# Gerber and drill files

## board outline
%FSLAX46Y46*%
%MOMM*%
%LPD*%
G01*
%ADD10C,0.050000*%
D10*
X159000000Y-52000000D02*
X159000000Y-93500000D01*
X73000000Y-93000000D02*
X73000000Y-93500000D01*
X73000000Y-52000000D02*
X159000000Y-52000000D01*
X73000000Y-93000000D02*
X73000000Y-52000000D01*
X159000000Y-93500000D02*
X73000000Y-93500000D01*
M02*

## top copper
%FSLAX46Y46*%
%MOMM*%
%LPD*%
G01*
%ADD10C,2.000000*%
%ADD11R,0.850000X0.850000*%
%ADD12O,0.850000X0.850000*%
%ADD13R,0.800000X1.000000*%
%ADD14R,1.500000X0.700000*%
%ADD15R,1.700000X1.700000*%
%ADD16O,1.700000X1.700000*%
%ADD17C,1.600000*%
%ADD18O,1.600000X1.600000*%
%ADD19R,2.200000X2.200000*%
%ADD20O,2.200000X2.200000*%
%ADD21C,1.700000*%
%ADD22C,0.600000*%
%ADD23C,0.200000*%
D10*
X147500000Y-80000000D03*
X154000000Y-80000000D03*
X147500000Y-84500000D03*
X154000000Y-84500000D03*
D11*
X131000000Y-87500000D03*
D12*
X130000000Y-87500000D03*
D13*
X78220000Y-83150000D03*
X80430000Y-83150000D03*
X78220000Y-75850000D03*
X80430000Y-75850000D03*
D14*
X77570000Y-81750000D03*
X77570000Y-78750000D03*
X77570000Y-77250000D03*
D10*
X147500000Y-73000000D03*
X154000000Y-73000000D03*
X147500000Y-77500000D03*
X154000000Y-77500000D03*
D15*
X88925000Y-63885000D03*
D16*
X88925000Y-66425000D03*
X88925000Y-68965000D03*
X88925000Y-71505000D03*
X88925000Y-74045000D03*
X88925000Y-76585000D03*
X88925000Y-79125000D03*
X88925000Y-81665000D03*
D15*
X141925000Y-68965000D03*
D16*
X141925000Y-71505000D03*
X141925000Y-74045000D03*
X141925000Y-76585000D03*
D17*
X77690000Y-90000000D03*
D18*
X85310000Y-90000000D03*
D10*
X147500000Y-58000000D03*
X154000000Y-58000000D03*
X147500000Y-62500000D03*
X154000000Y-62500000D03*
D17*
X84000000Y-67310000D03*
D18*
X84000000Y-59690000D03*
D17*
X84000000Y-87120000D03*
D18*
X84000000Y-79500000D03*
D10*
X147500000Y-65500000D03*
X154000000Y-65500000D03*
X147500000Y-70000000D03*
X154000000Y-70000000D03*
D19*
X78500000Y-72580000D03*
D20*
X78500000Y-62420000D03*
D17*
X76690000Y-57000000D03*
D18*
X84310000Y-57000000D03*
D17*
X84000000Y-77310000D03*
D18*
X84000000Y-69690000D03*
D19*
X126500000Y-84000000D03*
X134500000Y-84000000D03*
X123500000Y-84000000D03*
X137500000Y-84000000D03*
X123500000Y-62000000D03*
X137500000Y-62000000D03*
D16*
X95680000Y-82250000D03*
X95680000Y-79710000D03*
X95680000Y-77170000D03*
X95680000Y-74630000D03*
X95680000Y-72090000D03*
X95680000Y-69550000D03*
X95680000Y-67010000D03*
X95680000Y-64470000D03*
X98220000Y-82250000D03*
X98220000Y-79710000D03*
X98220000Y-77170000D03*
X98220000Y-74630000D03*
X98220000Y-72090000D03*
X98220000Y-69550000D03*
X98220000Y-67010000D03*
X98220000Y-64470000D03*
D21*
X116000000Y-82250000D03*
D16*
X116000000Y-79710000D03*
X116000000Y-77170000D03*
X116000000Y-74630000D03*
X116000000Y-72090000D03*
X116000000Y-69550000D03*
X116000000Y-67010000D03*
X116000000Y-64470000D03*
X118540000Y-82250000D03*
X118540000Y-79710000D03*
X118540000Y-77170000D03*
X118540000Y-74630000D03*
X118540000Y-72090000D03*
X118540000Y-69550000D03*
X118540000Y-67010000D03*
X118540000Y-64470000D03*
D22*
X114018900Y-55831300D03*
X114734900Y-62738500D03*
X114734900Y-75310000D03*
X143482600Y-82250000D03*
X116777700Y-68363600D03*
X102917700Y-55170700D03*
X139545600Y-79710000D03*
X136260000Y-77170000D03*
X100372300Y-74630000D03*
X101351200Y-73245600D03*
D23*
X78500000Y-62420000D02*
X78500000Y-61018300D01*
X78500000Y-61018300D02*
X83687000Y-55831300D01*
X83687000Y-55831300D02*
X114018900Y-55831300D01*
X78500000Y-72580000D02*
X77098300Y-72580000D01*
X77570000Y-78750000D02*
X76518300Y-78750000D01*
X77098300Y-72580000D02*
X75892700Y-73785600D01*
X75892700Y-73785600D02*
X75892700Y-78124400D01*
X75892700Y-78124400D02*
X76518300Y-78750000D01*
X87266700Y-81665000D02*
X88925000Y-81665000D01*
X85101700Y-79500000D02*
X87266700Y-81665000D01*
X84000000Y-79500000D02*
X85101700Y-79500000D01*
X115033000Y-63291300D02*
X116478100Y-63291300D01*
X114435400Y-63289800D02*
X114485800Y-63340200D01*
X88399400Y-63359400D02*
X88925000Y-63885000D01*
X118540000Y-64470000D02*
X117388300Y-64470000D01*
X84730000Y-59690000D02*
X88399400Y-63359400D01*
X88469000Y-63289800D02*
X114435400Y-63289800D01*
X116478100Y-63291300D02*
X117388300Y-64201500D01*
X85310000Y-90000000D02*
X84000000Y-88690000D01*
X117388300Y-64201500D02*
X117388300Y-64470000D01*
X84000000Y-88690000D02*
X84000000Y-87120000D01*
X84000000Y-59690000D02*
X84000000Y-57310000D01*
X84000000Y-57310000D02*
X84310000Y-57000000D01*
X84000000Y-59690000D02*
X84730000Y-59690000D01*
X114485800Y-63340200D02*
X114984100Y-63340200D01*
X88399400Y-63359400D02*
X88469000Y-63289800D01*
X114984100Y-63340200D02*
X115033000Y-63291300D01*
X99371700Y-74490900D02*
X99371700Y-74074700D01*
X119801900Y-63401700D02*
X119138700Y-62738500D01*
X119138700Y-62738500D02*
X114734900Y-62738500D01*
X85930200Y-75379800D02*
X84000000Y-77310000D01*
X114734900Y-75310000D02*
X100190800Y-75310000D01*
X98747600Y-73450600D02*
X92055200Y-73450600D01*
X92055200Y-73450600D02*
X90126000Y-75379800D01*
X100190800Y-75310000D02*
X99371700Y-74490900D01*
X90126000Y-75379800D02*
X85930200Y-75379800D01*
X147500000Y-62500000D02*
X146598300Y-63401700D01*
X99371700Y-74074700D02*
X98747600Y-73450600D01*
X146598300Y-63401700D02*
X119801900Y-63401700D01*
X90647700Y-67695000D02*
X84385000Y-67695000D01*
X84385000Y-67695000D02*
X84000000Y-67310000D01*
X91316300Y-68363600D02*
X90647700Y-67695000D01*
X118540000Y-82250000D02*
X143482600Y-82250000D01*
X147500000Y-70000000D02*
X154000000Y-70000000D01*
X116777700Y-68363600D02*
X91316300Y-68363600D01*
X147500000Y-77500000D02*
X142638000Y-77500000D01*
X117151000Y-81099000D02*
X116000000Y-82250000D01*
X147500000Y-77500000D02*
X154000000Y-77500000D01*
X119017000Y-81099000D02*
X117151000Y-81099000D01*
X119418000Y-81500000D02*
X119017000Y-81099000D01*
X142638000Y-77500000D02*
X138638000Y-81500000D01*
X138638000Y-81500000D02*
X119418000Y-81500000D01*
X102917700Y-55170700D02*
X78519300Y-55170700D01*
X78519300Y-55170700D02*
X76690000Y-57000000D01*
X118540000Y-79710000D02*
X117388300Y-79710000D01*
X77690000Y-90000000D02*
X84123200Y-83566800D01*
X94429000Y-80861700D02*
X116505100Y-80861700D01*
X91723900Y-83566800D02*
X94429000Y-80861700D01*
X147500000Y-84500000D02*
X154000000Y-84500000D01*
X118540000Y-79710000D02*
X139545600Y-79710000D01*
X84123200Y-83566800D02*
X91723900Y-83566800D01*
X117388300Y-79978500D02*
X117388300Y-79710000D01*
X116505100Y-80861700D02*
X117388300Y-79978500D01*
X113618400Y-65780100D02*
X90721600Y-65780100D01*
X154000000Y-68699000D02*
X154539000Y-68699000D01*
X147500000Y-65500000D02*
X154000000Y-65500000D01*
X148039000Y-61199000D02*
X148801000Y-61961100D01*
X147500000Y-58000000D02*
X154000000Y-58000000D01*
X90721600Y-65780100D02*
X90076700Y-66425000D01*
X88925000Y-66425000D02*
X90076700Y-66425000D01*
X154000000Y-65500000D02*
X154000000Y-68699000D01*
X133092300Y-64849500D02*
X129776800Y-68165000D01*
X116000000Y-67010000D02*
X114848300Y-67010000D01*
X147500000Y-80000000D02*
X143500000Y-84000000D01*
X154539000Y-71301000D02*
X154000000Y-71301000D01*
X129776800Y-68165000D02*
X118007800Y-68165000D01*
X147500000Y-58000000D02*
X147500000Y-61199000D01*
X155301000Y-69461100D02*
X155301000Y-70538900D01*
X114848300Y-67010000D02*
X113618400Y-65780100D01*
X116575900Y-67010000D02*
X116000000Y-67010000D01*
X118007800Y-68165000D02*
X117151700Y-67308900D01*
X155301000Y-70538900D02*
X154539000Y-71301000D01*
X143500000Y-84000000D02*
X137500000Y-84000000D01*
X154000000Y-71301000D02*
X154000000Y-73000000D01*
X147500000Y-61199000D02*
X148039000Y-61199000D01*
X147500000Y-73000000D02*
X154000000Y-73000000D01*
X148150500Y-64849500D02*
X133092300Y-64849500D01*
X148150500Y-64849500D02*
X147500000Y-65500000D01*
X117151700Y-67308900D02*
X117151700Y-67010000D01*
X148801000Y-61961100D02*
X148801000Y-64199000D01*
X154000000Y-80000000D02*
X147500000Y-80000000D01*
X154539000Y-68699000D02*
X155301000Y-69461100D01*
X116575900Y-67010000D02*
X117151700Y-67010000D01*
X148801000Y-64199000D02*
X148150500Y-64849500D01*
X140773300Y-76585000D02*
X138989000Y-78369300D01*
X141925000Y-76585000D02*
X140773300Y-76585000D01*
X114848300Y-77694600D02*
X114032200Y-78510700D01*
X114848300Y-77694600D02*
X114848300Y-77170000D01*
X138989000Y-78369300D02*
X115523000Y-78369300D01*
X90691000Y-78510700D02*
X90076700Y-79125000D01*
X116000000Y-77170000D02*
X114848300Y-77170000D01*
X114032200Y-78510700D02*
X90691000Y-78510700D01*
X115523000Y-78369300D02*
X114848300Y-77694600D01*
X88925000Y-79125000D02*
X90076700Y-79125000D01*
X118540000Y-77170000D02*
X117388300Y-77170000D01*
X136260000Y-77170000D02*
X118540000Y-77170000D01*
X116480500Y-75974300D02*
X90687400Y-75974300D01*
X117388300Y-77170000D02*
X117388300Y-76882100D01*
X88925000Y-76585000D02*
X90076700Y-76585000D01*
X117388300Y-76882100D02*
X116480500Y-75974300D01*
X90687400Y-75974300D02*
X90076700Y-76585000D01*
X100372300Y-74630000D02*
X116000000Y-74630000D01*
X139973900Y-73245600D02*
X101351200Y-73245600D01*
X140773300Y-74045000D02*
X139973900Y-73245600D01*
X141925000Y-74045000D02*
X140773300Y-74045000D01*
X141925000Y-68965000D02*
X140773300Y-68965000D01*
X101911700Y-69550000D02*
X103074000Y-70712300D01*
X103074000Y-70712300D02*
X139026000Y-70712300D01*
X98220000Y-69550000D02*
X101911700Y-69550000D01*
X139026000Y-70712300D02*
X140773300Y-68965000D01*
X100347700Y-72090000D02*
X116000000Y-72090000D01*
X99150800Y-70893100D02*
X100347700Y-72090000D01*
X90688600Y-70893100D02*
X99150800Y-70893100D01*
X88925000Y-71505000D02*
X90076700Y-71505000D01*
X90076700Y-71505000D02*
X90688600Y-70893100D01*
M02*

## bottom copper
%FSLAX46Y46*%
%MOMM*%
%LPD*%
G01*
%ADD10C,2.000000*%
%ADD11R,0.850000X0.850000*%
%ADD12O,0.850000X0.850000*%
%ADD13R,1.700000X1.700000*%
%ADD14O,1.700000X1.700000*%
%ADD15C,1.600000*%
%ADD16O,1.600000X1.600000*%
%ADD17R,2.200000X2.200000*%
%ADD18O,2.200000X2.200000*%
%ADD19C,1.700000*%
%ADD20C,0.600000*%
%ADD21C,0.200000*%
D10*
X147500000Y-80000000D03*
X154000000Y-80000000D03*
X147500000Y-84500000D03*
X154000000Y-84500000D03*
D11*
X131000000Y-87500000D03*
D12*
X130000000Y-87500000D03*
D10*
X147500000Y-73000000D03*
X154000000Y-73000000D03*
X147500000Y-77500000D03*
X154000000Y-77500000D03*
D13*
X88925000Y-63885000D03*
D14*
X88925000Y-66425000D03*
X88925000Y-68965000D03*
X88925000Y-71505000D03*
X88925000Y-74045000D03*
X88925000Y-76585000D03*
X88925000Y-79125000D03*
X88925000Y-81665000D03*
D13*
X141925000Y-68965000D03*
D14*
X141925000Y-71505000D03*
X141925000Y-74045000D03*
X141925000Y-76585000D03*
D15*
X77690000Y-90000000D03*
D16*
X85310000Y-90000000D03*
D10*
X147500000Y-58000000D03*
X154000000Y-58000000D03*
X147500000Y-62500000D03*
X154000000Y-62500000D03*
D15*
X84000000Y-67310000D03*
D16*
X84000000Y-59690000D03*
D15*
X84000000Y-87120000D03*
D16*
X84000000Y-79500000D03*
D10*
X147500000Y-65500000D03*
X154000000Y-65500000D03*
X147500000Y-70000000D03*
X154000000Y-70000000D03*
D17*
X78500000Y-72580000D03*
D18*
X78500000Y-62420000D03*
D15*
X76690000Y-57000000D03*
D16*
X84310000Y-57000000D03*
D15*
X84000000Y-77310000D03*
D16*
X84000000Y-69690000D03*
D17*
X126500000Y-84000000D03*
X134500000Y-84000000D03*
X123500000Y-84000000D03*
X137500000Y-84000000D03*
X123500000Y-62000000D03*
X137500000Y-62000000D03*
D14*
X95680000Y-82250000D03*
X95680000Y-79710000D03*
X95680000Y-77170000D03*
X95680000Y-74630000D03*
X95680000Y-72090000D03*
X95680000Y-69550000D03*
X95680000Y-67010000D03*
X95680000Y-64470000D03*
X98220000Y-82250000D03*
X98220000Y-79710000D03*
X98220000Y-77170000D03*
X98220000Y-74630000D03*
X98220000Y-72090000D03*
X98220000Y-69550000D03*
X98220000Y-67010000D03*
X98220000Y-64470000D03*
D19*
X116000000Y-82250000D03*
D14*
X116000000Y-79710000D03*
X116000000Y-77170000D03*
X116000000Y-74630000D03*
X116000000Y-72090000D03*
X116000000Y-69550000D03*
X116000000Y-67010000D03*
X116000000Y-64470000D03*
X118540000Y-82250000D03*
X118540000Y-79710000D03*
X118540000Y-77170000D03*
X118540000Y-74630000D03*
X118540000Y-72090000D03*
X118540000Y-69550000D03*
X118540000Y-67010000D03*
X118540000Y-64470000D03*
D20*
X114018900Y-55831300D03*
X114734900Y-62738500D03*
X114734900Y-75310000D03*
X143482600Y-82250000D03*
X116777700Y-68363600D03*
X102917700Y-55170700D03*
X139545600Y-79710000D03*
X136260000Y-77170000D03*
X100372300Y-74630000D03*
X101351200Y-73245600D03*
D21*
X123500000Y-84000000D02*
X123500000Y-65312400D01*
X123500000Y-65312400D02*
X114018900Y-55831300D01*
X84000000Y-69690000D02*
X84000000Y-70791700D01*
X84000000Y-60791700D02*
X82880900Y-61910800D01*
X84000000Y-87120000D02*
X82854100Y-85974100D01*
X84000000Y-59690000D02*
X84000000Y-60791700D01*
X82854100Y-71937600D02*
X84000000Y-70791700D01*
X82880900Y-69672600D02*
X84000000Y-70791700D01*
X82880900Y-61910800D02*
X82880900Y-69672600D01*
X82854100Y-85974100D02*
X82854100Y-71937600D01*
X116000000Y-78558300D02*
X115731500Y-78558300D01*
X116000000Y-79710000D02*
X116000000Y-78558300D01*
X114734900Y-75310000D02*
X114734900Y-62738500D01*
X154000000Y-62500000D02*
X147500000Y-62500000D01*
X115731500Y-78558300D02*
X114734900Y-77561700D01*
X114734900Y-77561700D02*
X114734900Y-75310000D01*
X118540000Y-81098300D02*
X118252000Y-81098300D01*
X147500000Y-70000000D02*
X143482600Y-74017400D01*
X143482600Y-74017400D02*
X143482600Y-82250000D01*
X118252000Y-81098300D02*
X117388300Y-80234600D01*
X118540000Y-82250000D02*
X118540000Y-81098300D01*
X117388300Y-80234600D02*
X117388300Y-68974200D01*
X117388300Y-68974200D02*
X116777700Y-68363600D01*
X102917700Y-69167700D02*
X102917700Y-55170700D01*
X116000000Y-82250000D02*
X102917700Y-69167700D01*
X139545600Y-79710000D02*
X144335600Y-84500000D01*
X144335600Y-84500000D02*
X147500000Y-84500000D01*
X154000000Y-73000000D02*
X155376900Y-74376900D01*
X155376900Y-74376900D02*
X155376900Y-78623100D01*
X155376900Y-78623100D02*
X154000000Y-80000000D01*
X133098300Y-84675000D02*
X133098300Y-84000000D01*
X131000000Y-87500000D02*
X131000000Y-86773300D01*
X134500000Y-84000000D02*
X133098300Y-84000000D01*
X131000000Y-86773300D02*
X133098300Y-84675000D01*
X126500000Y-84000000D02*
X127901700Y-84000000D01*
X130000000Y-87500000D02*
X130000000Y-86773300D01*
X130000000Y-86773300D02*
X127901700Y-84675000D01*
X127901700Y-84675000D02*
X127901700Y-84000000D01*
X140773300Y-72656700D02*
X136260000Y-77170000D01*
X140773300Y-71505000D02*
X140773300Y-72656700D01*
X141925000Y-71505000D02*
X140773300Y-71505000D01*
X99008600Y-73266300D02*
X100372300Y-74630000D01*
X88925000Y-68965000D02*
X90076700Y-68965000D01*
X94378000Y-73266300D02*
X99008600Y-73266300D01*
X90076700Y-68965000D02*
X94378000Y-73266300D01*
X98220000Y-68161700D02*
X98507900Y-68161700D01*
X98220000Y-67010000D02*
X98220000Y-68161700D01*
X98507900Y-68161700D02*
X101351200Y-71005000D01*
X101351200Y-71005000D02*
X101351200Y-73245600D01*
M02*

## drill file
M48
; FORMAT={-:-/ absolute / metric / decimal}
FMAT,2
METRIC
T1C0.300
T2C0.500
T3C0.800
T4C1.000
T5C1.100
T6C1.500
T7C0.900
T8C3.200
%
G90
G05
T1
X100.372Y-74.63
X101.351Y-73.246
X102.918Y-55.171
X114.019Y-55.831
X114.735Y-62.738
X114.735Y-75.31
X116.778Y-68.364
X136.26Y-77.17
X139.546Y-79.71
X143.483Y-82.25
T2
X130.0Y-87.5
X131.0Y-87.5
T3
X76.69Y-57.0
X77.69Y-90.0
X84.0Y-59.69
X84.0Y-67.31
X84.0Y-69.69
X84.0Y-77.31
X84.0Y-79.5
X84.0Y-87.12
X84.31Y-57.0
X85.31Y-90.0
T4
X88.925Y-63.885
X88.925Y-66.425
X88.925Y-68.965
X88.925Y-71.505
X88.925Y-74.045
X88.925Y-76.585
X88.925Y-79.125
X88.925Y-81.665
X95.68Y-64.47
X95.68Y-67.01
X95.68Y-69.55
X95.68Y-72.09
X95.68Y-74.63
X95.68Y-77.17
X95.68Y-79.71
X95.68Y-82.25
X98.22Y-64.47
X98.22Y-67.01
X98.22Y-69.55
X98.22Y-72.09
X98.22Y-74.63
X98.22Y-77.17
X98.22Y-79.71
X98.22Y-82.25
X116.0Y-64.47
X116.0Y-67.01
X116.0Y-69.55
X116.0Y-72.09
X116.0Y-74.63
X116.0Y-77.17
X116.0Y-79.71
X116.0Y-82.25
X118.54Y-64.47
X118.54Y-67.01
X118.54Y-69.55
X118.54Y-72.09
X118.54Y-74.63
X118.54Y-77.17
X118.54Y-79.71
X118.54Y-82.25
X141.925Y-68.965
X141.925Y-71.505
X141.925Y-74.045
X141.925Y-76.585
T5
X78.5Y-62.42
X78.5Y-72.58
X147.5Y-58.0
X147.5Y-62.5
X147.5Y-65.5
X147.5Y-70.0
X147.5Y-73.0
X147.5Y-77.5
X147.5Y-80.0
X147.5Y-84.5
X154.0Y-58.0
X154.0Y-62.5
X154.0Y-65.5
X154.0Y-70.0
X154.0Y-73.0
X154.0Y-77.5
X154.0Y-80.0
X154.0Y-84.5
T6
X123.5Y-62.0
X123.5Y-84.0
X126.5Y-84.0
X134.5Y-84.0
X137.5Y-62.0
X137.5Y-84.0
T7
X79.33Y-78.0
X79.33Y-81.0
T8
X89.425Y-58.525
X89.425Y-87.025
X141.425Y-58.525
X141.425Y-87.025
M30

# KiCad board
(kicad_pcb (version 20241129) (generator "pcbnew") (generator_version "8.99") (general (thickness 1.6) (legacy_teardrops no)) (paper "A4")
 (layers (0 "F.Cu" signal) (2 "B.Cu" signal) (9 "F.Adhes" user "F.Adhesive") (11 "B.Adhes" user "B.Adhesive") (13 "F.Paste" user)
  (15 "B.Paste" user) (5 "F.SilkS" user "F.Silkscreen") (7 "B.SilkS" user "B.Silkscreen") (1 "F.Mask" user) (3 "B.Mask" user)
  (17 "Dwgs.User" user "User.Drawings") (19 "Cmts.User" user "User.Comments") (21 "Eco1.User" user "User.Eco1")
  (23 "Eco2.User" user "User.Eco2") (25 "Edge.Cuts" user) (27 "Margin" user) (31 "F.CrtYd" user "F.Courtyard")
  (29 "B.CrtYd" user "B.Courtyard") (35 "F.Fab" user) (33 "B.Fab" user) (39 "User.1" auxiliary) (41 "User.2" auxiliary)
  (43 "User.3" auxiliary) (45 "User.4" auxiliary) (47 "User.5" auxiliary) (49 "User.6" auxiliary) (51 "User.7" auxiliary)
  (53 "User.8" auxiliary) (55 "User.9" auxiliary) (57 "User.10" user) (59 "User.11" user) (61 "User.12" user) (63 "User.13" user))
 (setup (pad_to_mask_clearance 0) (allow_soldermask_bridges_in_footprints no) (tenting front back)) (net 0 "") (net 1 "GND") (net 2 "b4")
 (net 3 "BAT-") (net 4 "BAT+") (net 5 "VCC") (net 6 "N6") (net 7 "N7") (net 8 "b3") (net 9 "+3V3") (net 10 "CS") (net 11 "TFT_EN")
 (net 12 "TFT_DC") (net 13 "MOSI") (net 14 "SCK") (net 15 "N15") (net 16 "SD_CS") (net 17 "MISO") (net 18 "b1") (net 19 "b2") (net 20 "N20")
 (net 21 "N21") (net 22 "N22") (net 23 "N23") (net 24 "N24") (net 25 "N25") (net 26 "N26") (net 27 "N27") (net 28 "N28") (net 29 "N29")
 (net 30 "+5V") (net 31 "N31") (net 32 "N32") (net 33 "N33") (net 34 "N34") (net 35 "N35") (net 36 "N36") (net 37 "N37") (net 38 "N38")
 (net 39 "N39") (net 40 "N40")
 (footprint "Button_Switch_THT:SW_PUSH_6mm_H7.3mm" (layer "F.Cu") (at 147.5 80)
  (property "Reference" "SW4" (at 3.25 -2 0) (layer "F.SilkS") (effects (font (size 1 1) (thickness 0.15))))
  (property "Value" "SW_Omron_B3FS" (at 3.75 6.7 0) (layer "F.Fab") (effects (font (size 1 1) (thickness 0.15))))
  (pad "1" thru_hole circle (at 0 0 90) (size 2 2) (drill 1.1) (layers "*.Cu" "*.Mask") (remove_unused_layers no) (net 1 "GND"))
  (pad "1" thru_hole circle (at 6.5 0 90) (size 2 2) (drill 1.1) (layers "*.Cu" "*.Mask") (remove_unused_layers no) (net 1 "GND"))
  (pad "2" thru_hole circle (at 0 4.5 90) (size 2 2) (drill 1.1) (layers "*.Cu" "*.Mask") (remove_unused_layers no) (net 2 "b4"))
  (pad "2" thru_hole circle (at 6.5 4.5 90) (size 2 2) (drill 1.1) (layers "*.Cu" "*.Mask") (remove_unused_layers no) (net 2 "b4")))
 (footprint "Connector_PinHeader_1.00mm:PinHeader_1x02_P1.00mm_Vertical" (layer "F.Cu") (at 131 87.5 -90)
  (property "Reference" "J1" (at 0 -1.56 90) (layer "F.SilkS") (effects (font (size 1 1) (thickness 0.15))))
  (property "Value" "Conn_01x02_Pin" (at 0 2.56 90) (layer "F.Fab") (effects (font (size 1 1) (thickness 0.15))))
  (pad "1" thru_hole rect (at 0 0 270) (size 0.85 0.85) (drill 0.5) (layers "*.Cu" "*.Mask") (remove_unused_layers no) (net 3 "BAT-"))
  (pad "2" thru_hole oval (at 0 1 270) (size 0.85 0.85) (drill 0.5) (layers "*.Cu" "*.Mask") (remove_unused_layers no) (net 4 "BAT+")))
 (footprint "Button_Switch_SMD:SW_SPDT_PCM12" (layer "F.Cu") (at 79 79.5 90)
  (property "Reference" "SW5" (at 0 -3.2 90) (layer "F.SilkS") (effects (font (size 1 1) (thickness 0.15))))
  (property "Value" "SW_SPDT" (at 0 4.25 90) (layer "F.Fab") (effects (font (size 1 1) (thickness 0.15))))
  (pad "" smd rect (at -3.65 -0.78 90) (size 1 0.8) (layers "F.Cu" "F.Mask" "F.Paste"))
  (pad "" smd rect (at -3.65 1.43 90) (size 1 0.8) (layers "F.Cu" "F.Mask" "F.Paste"))
  (pad "" np_thru_hole circle (at -1.5 0.33 90) (size 0.9 0.9) (drill 0.9) (layers "*.Cu" "*.Mask"))
  (pad "" np_thru_hole circle (at 1.5 0.33 90) (size 0.9 0.9) (drill 0.9) (layers "*.Cu" "*.Mask"))
  (pad "" smd rect (at 3.65 -0.78 90) (size 1 0.8) (layers "F.Cu" "F.Mask" "F.Paste"))
  (pad "" smd rect (at 3.65 1.43 90) (size 1 0.8) (layers "F.Cu" "F.Mask" "F.Paste"))
  (pad "1" smd rect (at -2.25 -1.43 90) (size 0.7 1.5) (layers "F.Cu" "F.Mask" "F.Paste") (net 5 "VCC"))
  (pad "2" smd rect (at 0.75 -1.43 90) (size 0.7 1.5) (layers "F.Cu" "F.Mask" "F.Paste") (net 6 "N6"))
  (pad "3" smd rect (at 2.25 -1.43 90) (size 0.7 1.5) (layers "F.Cu" "F.Mask" "F.Paste") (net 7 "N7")))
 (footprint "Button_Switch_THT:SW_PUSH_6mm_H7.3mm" (layer "F.Cu") (at 147.5 73)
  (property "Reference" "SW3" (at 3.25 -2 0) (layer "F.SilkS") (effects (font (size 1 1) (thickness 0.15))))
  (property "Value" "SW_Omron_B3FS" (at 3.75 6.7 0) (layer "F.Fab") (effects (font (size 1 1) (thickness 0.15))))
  (pad "1" thru_hole circle (at 0 0 90) (size 2 2) (drill 1.1) (layers "*.Cu" "*.Mask") (remove_unused_layers no) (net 1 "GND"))
  (pad "1" thru_hole circle (at 6.5 0 90) (size 2 2) (drill 1.1) (layers "*.Cu" "*.Mask") (remove_unused_layers no) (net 1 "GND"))
  (pad "2" thru_hole circle (at 0 4.5 90) (size 2 2) (drill 1.1) (layers "*.Cu" "*.Mask") (remove_unused_layers no) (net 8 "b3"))
  (pad "2" thru_hole circle (at 6.5 4.5 90) (size 2 2) (drill 1.1) (layers "*.Cu" "*.Mask") (remove_unused_layers no) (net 8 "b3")))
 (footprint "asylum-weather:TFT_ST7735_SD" (layer "F.Cu") (at 108.925 72.525)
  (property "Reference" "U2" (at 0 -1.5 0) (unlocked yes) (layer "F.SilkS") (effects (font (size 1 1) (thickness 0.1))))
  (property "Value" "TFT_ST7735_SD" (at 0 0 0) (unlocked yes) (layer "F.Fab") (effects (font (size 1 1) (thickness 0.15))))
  (pad "" np_thru_hole circle (at -19.5 -14) (size 3.2 3.2) (drill 3.2) (layers "*.Cu" "*.Mask"))
  (pad "" np_thru_hole circle (at -19.5 14.5) (size 3.2 3.2) (drill 3.2) (layers "*.Cu" "*.Mask"))
  (pad "" np_thru_hole circle (at 32.5 -14) (size 3.2 3.2) (drill 3.2) (layers "*.Cu" "*.Mask"))
  (pad "" np_thru_hole circle (at 32.5 14.5) (size 3.2 3.2) (drill 3.2) (layers "*.Cu" "*.Mask"))
  (pad "1" thru_hole rect (at -20 -8.64) (size 1.7 1.7) (drill 1) (layers "*.Cu" "*.Mask") (remove_unused_layers no) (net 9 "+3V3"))
  (pad "2" thru_hole oval (at -20 -6.1) (size 1.7 1.7) (drill 1) (layers "*.Cu" "*.Mask") (remove_unused_layers no) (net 1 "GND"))
  (pad "3" thru_hole oval (at -20 -3.56) (size 1.7 1.7) (drill 1) (layers "*.Cu" "*.Mask") (remove_unused_layers no) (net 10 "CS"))
  (pad "4" thru_hole oval (at -20 -1.02) (size 1.7 1.7) (drill 1) (layers "*.Cu" "*.Mask") (remove_unused_layers no) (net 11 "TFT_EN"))
  (pad "5" thru_hole oval (at -20 1.52) (size 1.7 1.7) (drill 1) (layers "*.Cu" "*.Mask") (remove_unused_layers no) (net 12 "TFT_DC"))
  (pad "6" thru_hole oval (at -20 4.06) (size 1.7 1.7) (drill 1) (layers "*.Cu" "*.Mask") (remove_unused_layers no) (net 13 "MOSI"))
  (pad "7" thru_hole oval (at -20 6.6) (size 1.7 1.7) (drill 1) (layers "*.Cu" "*.Mask") (remove_unused_layers no) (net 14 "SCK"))
  (pad "8" thru_hole oval (at -20 9.14) (size 1.7 1.7) (drill 1) (layers "*.Cu" "*.Mask") (remove_unused_layers no) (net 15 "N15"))
  (pad "9" thru_hole rect (at 33 -3.56) (size 1.7 1.7) (drill 1) (layers "*.Cu" "*.Mask") (remove_unused_layers no) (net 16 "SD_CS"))
  (pad "10" thru_hole oval (at 33 -1.02) (size 1.7 1.7) (drill 1) (layers "*.Cu" "*.Mask") (remove_unused_layers no) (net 13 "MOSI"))
  (pad "11" thru_hole oval (at 33 1.52) (size 1.7 1.7) (drill 1) (layers "*.Cu" "*.Mask") (remove_unused_layers no) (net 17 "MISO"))
  (pad "12" thru_hole oval (at 33 4.06) (size 1.7 1.7) (drill 1) (layers "*.Cu" "*.Mask") (remove_unused_layers no) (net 14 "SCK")))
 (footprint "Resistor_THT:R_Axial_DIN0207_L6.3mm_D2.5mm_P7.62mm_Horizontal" (layer "F.Cu") (at 77.69 90)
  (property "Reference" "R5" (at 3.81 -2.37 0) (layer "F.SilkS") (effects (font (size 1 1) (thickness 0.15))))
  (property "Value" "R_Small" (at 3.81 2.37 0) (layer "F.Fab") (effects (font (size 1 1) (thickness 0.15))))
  (pad "1" thru_hole circle (at 0 0) (size 1.6 1.6) (drill 0.8) (layers "*.Cu" "*.Mask") (remove_unused_layers no) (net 2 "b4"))
  (pad "2" thru_hole oval (at 7.62 0) (size 1.6 1.6) (drill 0.8) (layers "*.Cu" "*.Mask") (remove_unused_layers no) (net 9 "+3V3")))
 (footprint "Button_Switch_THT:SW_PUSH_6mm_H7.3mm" (layer "F.Cu") (at 147.5 58)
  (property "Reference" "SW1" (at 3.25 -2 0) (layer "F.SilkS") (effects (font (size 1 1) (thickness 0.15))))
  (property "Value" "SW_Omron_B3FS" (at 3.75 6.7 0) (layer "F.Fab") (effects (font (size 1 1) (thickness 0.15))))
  (pad "1" thru_hole circle (at 0 0 90) (size 2 2) (drill 1.1) (layers "*.Cu" "*.Mask") (remove_unused_layers no) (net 1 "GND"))
  (pad "1" thru_hole circle (at 6.5 0 90) (size 2 2) (drill 1.1) (layers "*.Cu" "*.Mask") (remove_unused_layers no) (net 1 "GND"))
  (pad "2" thru_hole circle (at 0 4.5 90) (size 2 2) (drill 1.1) (layers "*.Cu" "*.Mask") (remove_unused_layers no) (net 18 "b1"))
  (pad "2" thru_hole circle (at 6.5 4.5 90) (size 2 2) (drill 1.1) (layers "*.Cu" "*.Mask") (remove_unused_layers no) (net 18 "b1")))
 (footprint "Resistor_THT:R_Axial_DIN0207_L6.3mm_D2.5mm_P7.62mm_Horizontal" (layer "F.Cu") (at 84 67.31 90)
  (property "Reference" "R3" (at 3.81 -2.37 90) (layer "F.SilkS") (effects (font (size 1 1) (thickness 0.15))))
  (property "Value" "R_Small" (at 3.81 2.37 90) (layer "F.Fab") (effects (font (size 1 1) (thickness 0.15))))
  (pad "1" thru_hole circle (at 0 0 90) (size 1.6 1.6) (drill 0.8) (layers "*.Cu" "*.Mask") (remove_unused_layers no) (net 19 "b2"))
  (pad "2" thru_hole oval (at 7.62 0 90) (size 1.6 1.6) (drill 0.8) (layers "*.Cu" "*.Mask") (remove_unused_layers no) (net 9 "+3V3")))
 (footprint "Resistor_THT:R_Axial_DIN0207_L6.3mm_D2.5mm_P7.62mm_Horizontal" (layer "F.Cu") (at 84 87.12 90)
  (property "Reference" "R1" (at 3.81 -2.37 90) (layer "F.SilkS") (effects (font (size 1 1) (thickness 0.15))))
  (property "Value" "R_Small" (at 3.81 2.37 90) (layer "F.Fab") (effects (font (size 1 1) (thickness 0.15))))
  (pad "1" thru_hole circle (at 0 0 90) (size 1.6 1.6) (drill 0.8) (layers "*.Cu" "*.Mask") (remove_unused_layers no) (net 9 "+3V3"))
  (pad "2" thru_hole oval (at 7.62 0 90) (size 1.6 1.6) (drill 0.8) (layers "*.Cu" "*.Mask") (remove_unused_layers no) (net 15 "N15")))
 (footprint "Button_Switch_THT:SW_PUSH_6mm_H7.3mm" (layer "F.Cu") (at 147.5 65.5)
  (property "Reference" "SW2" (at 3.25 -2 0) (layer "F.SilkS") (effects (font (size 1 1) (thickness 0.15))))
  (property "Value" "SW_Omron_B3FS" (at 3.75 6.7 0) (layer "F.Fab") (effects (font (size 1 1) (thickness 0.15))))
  (pad "1" thru_hole circle (at 0 0 90) (size 2 2) (drill 1.1) (layers "*.Cu" "*.Mask") (remove_unused_layers no) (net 1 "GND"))
  (pad "1" thru_hole circle (at 6.5 0 90) (size 2 2) (drill 1.1) (layers "*.Cu" "*.Mask") (remove_unused_layers no) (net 1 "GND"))
  (pad "2" thru_hole circle (at 0 4.5 90) (size 2 2) (drill 1.1) (layers "*.Cu" "*.Mask") (remove_unused_layers no) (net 19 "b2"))
  (pad "2" thru_hole circle (at 6.5 4.5 90) (size 2 2) (drill 1.1) (layers "*.Cu" "*.Mask") (remove_unused_layers no) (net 19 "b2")))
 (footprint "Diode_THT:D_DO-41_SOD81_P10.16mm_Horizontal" (layer "F.Cu") (at 78.5 72.58 90)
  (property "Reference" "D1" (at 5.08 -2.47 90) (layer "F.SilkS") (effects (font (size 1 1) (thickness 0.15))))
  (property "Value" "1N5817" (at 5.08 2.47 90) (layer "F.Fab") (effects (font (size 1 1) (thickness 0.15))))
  (pad "1" thru_hole rect (at 0 0 90) (size 2.2 2.2) (drill 1.1) (layers "*.Cu" "*.Mask") (remove_unused_layers no) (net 6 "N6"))
  (pad "2" thru_hole oval (at 10.16 0 90) (size 2.2 2.2) (drill 1.1) (layers "*.Cu" "*.Mask") (remove_unused_layers no) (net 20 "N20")))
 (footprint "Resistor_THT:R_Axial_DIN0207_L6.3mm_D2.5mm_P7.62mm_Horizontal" (layer "F.Cu") (at 76.69 57)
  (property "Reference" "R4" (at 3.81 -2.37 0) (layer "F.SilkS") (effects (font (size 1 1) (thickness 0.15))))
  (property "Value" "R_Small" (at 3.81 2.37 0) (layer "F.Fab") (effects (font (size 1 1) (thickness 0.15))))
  (pad "1" thru_hole circle (at 0 0) (size 1.6 1.6) (drill 0.8) (layers "*.Cu" "*.Mask") (remove_unused_layers no) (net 8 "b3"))
  (pad "2" thru_hole oval (at 7.62 0) (size 1.6 1.6) (drill 0.8) (layers "*.Cu" "*.Mask") (remove_unused_layers no) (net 9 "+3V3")))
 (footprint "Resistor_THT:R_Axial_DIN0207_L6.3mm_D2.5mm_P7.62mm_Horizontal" (layer "F.Cu") (at 84 77.31 90)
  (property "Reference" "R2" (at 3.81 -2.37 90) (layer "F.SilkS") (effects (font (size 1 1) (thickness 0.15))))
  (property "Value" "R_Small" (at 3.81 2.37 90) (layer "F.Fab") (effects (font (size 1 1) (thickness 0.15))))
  (pad "1" thru_hole circle (at 0 0 90) (size 1.6 1.6) (drill 0.8) (layers "*.Cu" "*.Mask") (remove_unused_layers no) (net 18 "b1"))
  (pad "2" thru_hole oval (at 7.62 0 90) (size 1.6 1.6) (drill 0.8) (layers "*.Cu" "*.Mask") (remove_unused_layers no) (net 9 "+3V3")))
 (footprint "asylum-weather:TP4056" (layer "B.Cu") (at 130.5 73.5 180)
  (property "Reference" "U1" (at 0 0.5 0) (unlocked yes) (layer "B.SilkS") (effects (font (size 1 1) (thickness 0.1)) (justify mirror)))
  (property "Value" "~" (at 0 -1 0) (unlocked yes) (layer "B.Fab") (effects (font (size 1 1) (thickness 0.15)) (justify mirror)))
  (pad "0" thru_hole rect (at 4 -10.5 90) (size 2.2 2.2) (drill 1.5) (layers "F&B.Cu" "*.Mask") (remove_unused_layers no) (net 4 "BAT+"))
  (pad "1" thru_hole rect (at -4 -10.5 90) (size 2.2 2.2) (drill 1.5) (layers "F&B.Cu" "*.Mask") (remove_unused_layers no) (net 3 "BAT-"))
  (pad "2" thru_hole rect (at 7 -10.5 90) (size 2.2 2.2) (drill 1.5) (layers "F&B.Cu" "*.Mask") (remove_unused_layers no) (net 20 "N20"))
  (pad "3" thru_hole rect (at -7 -10.5 90) (size 2.2 2.2) (drill 1.5) (layers "F&B.Cu" "*.Mask") (remove_unused_layers no) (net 1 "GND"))
  (pad "4" thru_hole rect (at 7 11.5 90) (size 2.2 2.2) (drill 1.5) (layers "F&B.Cu" "*.Mask") (remove_unused_layers no) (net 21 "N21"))
  (pad "5" thru_hole rect (at -7 11.5 90) (size 2.2 2.2) (drill 1.5) (layers "F&B.Cu" "*.Mask") (remove_unused_layers no) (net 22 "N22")))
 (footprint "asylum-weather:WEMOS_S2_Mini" (layer "B.Cu") (at 107.11 74.75)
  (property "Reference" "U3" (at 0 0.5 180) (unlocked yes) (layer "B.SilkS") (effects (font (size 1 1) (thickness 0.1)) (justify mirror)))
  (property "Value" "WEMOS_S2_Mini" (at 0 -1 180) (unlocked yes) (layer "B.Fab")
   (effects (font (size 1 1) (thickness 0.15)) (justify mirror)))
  (pad "1" thru_hole oval (at -11.43 7.5) (size 1.7 1.7) (drill 1) (layers "F&B.Cu" "*.Mask") (remove_unused_layers no) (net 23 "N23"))
  (pad "2" thru_hole oval (at -11.43 4.96) (size 1.7 1.7) (drill 1) (layers "F&B.Cu" "*.Mask") (remove_unused_layers no) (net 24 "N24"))
  (pad "3" thru_hole oval (at -11.43 2.42) (size 1.7 1.7) (drill 1) (layers "F&B.Cu" "*.Mask") (remove_unused_layers no) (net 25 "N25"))
  (pad "4" thru_hole oval (at -11.43 -0.12) (size 1.7 1.7) (drill 1) (layers "F&B.Cu" "*.Mask") (remove_unused_layers no) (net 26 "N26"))
  (pad "5" thru_hole oval (at -11.43 -2.66) (size 1.7 1.7) (drill 1) (layers "F&B.Cu" "*.Mask") (remove_unused_layers no) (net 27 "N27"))
  (pad "6" thru_hole oval (at -11.43 -5.2) (size 1.7 1.7) (drill 1) (layers "F&B.Cu" "*.Mask") (remove_unused_layers no) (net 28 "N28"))
  (pad "7" thru_hole oval (at -11.43 -7.74) (size 1.7 1.7) (drill 1) (layers "F&B.Cu" "*.Mask") (remove_unused_layers no) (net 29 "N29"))
  (pad "8" thru_hole oval (at -11.43 -10.28) (size 1.7 1.7) (drill 1) (layers "F&B.Cu" "*.Mask") (remove_unused_layers no) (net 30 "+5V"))
  (pad "9" thru_hole oval (at -8.89 7.5) (size 1.7 1.7) (drill 1) (layers "F&B.Cu" "*.Mask") (remove_unused_layers no) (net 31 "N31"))
  (pad "10" thru_hole oval (at -8.89 4.96) (size 1.7 1.7) (drill 1) (layers "F&B.Cu" "*.Mask") (remove_unused_layers no) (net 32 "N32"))
  (pad "11" thru_hole oval (at -8.89 2.42) (size 1.7 1.7) (drill 1) (layers "F&B.Cu" "*.Mask") (remove_unused_layers no) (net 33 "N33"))
  (pad "12" thru_hole oval (at -8.89 -0.12) (size 1.7 1.7) (drill 1) (layers "F&B.Cu" "*.Mask") (remove_unused_layers no) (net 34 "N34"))
  (pad "13" thru_hole oval (at -8.89 -2.66) (size 1.7 1.7) (drill 1) (layers "F&B.Cu" "*.Mask") (remove_unused_layers no) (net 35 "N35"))
  (pad "14" thru_hole oval (at -8.89 -5.2) (size 1.7 1.7) (drill 1) (layers "F&B.Cu" "*.Mask") (remove_unused_layers no) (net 16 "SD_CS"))
  (pad "15" thru_hole oval (at -8.89 -7.74) (size 1.7 1.7) (drill 1) (layers "F&B.Cu" "*.Mask") (remove_unused_layers no) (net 17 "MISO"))
  (pad "16" thru_hole oval (at -8.89 -10.28) (size 1.7 1.7) (drill 1) (layers "F&B.Cu" "*.Mask") (remove_unused_layers no) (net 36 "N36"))
  (pad "17" thru_hole circle (at 8.89 7.5) (size 1.7 1.7) (drill 1) (layers "F&B.Cu" "*.Mask") (remove_unused_layers no) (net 8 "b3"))
  (pad "18" thru_hole oval (at 8.89 4.96) (size 1.7 1.7) (drill 1) (layers "F&B.Cu" "*.Mask") (remove_unused_layers no) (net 18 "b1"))
  (pad "19" thru_hole oval (at 8.89 2.42) (size 1.7 1.7) (drill 1) (layers "F&B.Cu" "*.Mask") (remove_unused_layers no) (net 14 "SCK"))
  (pad "20" thru_hole oval (at 8.89 -0.12) (size 1.7 1.7) (drill 1) (layers "F&B.Cu" "*.Mask") (remove_unused_layers no) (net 10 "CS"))
  (pad "21" thru_hole oval (at 8.89 -2.66) (size 1.7 1.7) (drill 1) (layers "F&B.Cu" "*.Mask") (remove_unused_layers no) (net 11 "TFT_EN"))
  (pad "22" thru_hole oval (at 8.89 -5.2) (size 1.7 1.7) (drill 1) (layers "F&B.Cu" "*.Mask") (remove_unused_layers no) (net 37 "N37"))
  (pad "23" thru_hole oval (at 8.89 -7.74) (size 1.7 1.7) (drill 1) (layers "F&B.Cu" "*.Mask") (remove_unused_layers no) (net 1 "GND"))
  (pad "24" thru_hole oval (at 8.89 -10.28) (size 1.7 1.7) (drill 1) (layers "F&B.Cu" "*.Mask") (remove_unused_layers no) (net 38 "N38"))
  (pad "25" thru_hole oval (at 11.43 7.5) (size 1.7 1.7) (drill 1) (layers "F&B.Cu" "*.Mask") (remove_unused_layers no) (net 19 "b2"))
  (pad "26" thru_hole oval (at 11.43 4.96) (size 1.7 1.7) (drill 1) (layers "F&B.Cu" "*.Mask") (remove_unused_layers no) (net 2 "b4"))
  (pad "27" thru_hole oval (at 11.43 2.42) (size 1.7 1.7) (drill 1) (layers "F&B.Cu" "*.Mask") (remove_unused_layers no) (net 13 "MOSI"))
  (pad "28" thru_hole oval (at 11.43 -0.12) (size 1.7 1.7) (drill 1) (layers "F&B.Cu" "*.Mask") (remove_unused_layers no) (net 12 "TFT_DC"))
  (pad "29" thru_hole oval (at 11.43 -2.66) (size 1.7 1.7) (drill 1) (layers "F&B.Cu" "*.Mask") (remove_unused_layers no) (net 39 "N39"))
  (pad "30" thru_hole oval (at 11.43 -5.2) (size 1.7 1.7) (drill 1) (layers "F&B.Cu" "*.Mask") (remove_unused_layers no) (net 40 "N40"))
  (pad "31" thru_hole oval (at 11.43 -7.74) (size 1.7 1.7) (drill 1) (layers "F&B.Cu" "*.Mask") (remove_unused_layers no))
  (pad "32" thru_hole oval (at 11.43 -10.28) (size 1.7 1.7) (drill 1) (layers "F&B.Cu" "*.Mask") (remove_unused_layers no) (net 9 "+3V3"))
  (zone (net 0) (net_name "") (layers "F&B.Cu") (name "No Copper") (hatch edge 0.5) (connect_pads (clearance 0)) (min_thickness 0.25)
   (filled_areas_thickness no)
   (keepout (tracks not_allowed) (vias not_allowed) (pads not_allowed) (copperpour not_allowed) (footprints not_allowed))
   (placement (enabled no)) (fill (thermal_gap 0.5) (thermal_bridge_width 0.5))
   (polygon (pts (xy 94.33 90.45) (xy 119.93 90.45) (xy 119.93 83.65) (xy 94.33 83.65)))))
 (gr_line (start 159 52) (end 159 93.5) (stroke (width 0.05) (type default)) (layer "Edge.Cuts"))
 (gr_line (start 73 93) (end 73 93.5) (stroke (width 0.05) (type default)) (layer "Edge.Cuts"))
 (gr_line (start 73 52) (end 159 52) (stroke (width 0.05) (type default)) (layer "Edge.Cuts"))
 (gr_line (start 73 93) (end 73 52) (stroke (width 0.05) (type default)) (layer "Edge.Cuts"))
 (gr_line (start 159 93.5) (end 73 93.5) (stroke (width 0.05) (type default)) (layer "Edge.Cuts"))
 (segment (start 78.5 62.42) (end 78.5 61.0183) (width 0.2) (layer "F.Cu") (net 20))
 (segment (start 78.5 61.0183) (end 83.687 55.8313) (width 0.2) (layer "F.Cu") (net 20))
 (segment (start 83.687 55.8313) (end 114.0189 55.8313) (width 0.2) (layer "F.Cu") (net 20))
 (via (at 114.0189 55.8313) (size 0.6) (drill 0.3) (layers "F.Cu" "B.Cu") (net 20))
 (segment (start 123.5 84) (end 123.5 65.3124) (width 0.2) (layer "B.Cu") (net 20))
 (segment (start 123.5 65.3124) (end 114.0189 55.8313) (width 0.2) (layer "B.Cu") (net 20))
 (segment (start 78.5 72.58) (end 77.0983 72.58) (width 0.2) (layer "F.Cu") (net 6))
 (segment (start 77.57 78.75) (end 76.5183 78.75) (width 0.2) (layer "F.Cu") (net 6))
 (segment (start 77.0983 72.58) (end 75.8927 73.7856) (width 0.2) (layer "F.Cu") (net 6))
 (segment (start 75.8927 73.7856) (end 75.8927 78.1244) (width 0.2) (layer "F.Cu") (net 6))
 (segment (start 75.8927 78.1244) (end 76.5183 78.75) (width 0.2) (layer "F.Cu") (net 6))
 (segment (start 87.2667 81.665) (end 88.925 81.665) (width 0.2) (layer "F.Cu") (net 15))
 (segment (start 85.1017 79.5) (end 87.2667 81.665) (width 0.2) (layer "F.Cu") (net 15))
 (segment (start 84 79.5) (end 85.1017 79.5) (width 0.2) (layer "F.Cu") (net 15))
 (segment (start 115.033 63.2913) (end 116.4781 63.2913) (width 0.2) (layer "F.Cu") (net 9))
 (segment (start 114.4354 63.2898) (end 114.4858 63.3402) (width 0.2) (layer "F.Cu") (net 9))
 (segment (start 88.3994 63.3594) (end 88.925 63.885) (width 0.2) (layer "F.Cu") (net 9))
 (segment (start 118.54 64.47) (end 117.3883 64.47) (width 0.2) (layer "F.Cu") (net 9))
 (segment (start 84.73 59.69) (end 88.3994 63.3594) (width 0.2) (layer "F.Cu") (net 9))
 (segment (start 88.469 63.2898) (end 114.4354 63.2898) (width 0.2) (layer "F.Cu") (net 9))
 (segment (start 116.4781 63.2913) (end 117.3883 64.2015) (width 0.2) (layer "F.Cu") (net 9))
 (segment (start 85.31 90) (end 84 88.69) (width 0.2) (layer "F.Cu") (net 9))
 (segment (start 117.3883 64.2015) (end 117.3883 64.47) (width 0.2) (layer "F.Cu") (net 9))
 (segment (start 84 88.69) (end 84 87.12) (width 0.2) (layer "F.Cu") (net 9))
 (segment (start 84 59.69) (end 84 57.31) (width 0.2) (layer "F.Cu") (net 9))
 (segment (start 84 57.31) (end 84.31 57) (width 0.2) (layer "F.Cu") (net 9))
 (segment (start 84 59.69) (end 84.73 59.69) (width 0.2) (layer "F.Cu") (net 9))
 (segment (start 114.4858 63.3402) (end 114.9841 63.3402) (width 0.2) (layer "F.Cu") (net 9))
 (segment (start 88.3994 63.3594) (end 88.469 63.2898) (width 0.2) (layer "F.Cu") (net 9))
 (segment (start 114.9841 63.3402) (end 115.033 63.2913) (width 0.2) (layer "F.Cu") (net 9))
 (segment (start 84 69.69) (end 84 70.7917) (width 0.2) (layer "B.Cu") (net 9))
 (segment (start 84 60.7917) (end 82.8809 61.9108) (width 0.2) (layer "B.Cu") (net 9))
 (segment (start 84 87.12) (end 82.8541 85.9741) (width 0.2) (layer "B.Cu") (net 9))
 (segment (start 84 59.69) (end 84 60.7917) (width 0.2) (layer "B.Cu") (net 9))
 (segment (start 82.8541 71.9376) (end 84 70.7917) (width 0.2) (layer "B.Cu") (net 9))
 (segment (start 82.8809 69.6726) (end 84 70.7917) (width 0.2) (layer "B.Cu") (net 9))
 (segment (start 82.8809 61.9108) (end 82.8809 69.6726) (width 0.2) (layer "B.Cu") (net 9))
 (segment (start 82.8541 85.9741) (end 82.8541 71.9376) (width 0.2) (layer "B.Cu") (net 9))
 (segment (start 99.3717 74.4909) (end 99.3717 74.0747) (width 0.2) (layer "F.Cu") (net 18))
 (segment (start 119.8019 63.4017) (end 119.1387 62.7385) (width 0.2) (layer "F.Cu") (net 18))
 (segment (start 119.1387 62.7385) (end 114.7349 62.7385) (width 0.2) (layer "F.Cu") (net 18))
 (segment (start 85.9302 75.3798) (end 84 77.31) (width 0.2) (layer "F.Cu") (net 18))
 (segment (start 114.7349 75.31) (end 100.1908 75.31) (width 0.2) (layer "F.Cu") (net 18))
 (segment (start 98.7476 73.4506) (end 92.0552 73.4506) (width 0.2) (layer "F.Cu") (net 18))
 (segment (start 92.0552 73.4506) (end 90.126 75.3798) (width 0.2) (layer "F.Cu") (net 18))
 (segment (start 100.1908 75.31) (end 99.3717 74.4909) (width 0.2) (layer "F.Cu") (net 18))
 (segment (start 90.126 75.3798) (end 85.9302 75.3798) (width 0.2) (layer "F.Cu") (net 18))
 (segment (start 147.5 62.5) (end 146.5983 63.4017) (width 0.2) (layer "F.Cu") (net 18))
 (segment (start 99.3717 74.0747) (end 98.7476 73.4506) (width 0.2) (layer "F.Cu") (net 18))
 (segment (start 146.5983 63.4017) (end 119.8019 63.4017) (width 0.2) (layer "F.Cu") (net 18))
 (via (at 114.7349 62.7385) (size 0.6) (drill 0.3) (layers "F.Cu" "B.Cu") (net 18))
 (via (at 114.7349 75.31) (size 0.6) (drill 0.3) (layers "F.Cu" "B.Cu") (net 18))
 (segment (start 116 78.5583) (end 115.7315 78.5583) (width 0.2) (layer "B.Cu") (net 18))
 (segment (start 116 79.71) (end 116 78.5583) (width 0.2) (layer "B.Cu") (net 18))
 (segment (start 114.7349 75.31) (end 114.7349 62.7385) (width 0.2) (layer "B.Cu") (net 18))
 (segment (start 154 62.5) (end 147.5 62.5) (width 0.2) (layer "B.Cu") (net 18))
 (segment (start 115.7315 78.5583) (end 114.7349 77.5617) (width 0.2) (layer "B.Cu") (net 18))
 (segment (start 114.7349 77.5617) (end 114.7349 75.31) (width 0.2) (layer "B.Cu") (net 18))
 (segment (start 90.6477 67.695) (end 84.385 67.695) (width 0.2) (layer "F.Cu") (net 19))
 (segment (start 84.385 67.695) (end 84 67.31) (width 0.2) (layer "F.Cu") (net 19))
 (segment (start 91.3163 68.3636) (end 90.6477 67.695) (width 0.2) (layer "F.Cu") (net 19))
 (segment (start 118.54 82.25) (end 143.4826 82.25) (width 0.2) (layer "F.Cu") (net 19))
 (segment (start 147.5 70) (end 154 70) (width 0.2) (layer "F.Cu") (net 19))
 (segment (start 116.7777 68.3636) (end 91.3163 68.3636) (width 0.2) (layer "F.Cu") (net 19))
 (via (at 143.4826 82.25) (size 0.6) (drill 0.3) (layers "F.Cu" "B.Cu") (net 19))
 (via (at 116.7777 68.3636) (size 0.6) (drill 0.3) (layers "F.Cu" "B.Cu") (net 19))
 (segment (start 118.54 81.0983) (end 118.252 81.0983) (width 0.2) (layer "B.Cu") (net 19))
 (segment (start 147.5 70) (end 143.4826 74.0174) (width 0.2) (layer "B.Cu") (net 19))
 (segment (start 143.4826 74.0174) (end 143.4826 82.25) (width 0.2) (layer "B.Cu") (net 19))
 (segment (start 118.252 81.0983) (end 117.3883 80.2346) (width 0.2) (layer "B.Cu") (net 19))
 (segment (start 118.54 82.25) (end 118.54 81.0983) (width 0.2) (layer "B.Cu") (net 19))
 (segment (start 117.3883 80.2346) (end 117.3883 68.9742) (width 0.2) (layer "B.Cu") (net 19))
 (segment (start 117.3883 68.9742) (end 116.7777 68.3636) (width 0.2) (layer "B.Cu") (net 19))
 (segment (start 147.5 77.5) (end 142.638 77.5) (width 0.2) (layer "F.Cu") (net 8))
 (segment (start 117.151 81.099) (end 116 82.25) (width 0.2) (layer "F.Cu") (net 8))
 (segment (start 147.5 77.5) (end 154 77.5) (width 0.2) (layer "F.Cu") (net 8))
 (segment (start 119.017 81.099) (end 117.151 81.099) (width 0.2) (layer "F.Cu") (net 8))
 (segment (start 119.418 81.5) (end 119.017 81.099) (width 0.2) (layer "F.Cu") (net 8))
 (segment (start 142.638 77.5) (end 138.638 81.5) (width 0.2) (layer "F.Cu") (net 8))
 (segment (start 138.638 81.5) (end 119.418 81.5) (width 0.2) (layer "F.Cu") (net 8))
 (segment (start 102.9177 55.1707) (end 78.5193 55.1707) (width 0.2) (layer "F.Cu") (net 8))
 (segment (start 78.5193 55.1707) (end 76.69 57) (width 0.2) (layer "F.Cu") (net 8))
 (via (at 102.9177 55.1707) (size 0.6) (drill 0.3) (layers "F.Cu" "B.Cu") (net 8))
 (segment (start 102.9177 69.1677) (end 102.9177 55.1707) (width 0.2) (layer "B.Cu") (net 8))
 (segment (start 116 82.25) (end 102.9177 69.1677) (width 0.2) (layer "B.Cu") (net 8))
 (segment (start 118.54 79.71) (end 117.3883 79.71) (width 0.2) (layer "F.Cu") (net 2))
 (segment (start 77.69 90) (end 84.1232 83.5668) (width 0.2) (layer "F.Cu") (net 2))
 (segment (start 94.429 80.8617) (end 116.5051 80.8617) (width 0.2) (layer "F.Cu") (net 2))
 (segment (start 91.7239 83.5668) (end 94.429 80.8617) (width 0.2) (layer "F.Cu") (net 2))
 (segment (start 147.5 84.5) (end 154 84.5) (width 0.2) (layer "F.Cu") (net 2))
 (segment (start 118.54 79.71) (end 139.5456 79.71) (width 0.2) (layer "F.Cu") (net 2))
 (segment (start 84.1232 83.5668) (end 91.7239 83.5668) (width 0.2) (layer "F.Cu") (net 2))
 (segment (start 117.3883 79.9785) (end 117.3883 79.71) (width 0.2) (layer "F.Cu") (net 2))
 (segment (start 116.5051 80.8617) (end 117.3883 79.9785) (width 0.2) (layer "F.Cu") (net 2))
 (via (at 139.5456 79.71) (size 0.6) (drill 0.3) (layers "F.Cu" "B.Cu") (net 2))
 (segment (start 139.5456 79.71) (end 144.3356 84.5) (width 0.2) (layer "B.Cu") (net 2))
 (segment (start 144.3356 84.5) (end 147.5 84.5) (width 0.2) (layer "B.Cu") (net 2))
 (segment (start 113.6184 65.7801) (end 90.7216 65.7801) (width 0.2) (layer "F.Cu") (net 1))
 (segment (start 154 68.699) (end 154.539 68.699) (width 0.2) (layer "F.Cu") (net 1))
 (segment (start 147.5 65.5) (end 154 65.5) (width 0.2) (layer "F.Cu") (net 1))
 (segment (start 148.039 61.199) (end 148.801 61.9611) (width 0.2) (layer "F.Cu") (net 1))
 (segment (start 147.5 58) (end 154 58) (width 0.2) (layer "F.Cu") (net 1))
 (segment (start 90.7216 65.7801) (end 90.0767 66.425) (width 0.2) (layer "F.Cu") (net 1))
 (segment (start 88.925 66.425) (end 90.0767 66.425) (width 0.2) (layer "F.Cu") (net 1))
 (segment (start 154 65.5) (end 154 68.699) (width 0.2) (layer "F.Cu") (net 1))
 (segment (start 133.0923 64.8495) (end 129.7768 68.165) (width 0.2) (layer "F.Cu") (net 1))
 (segment (start 116 67.01) (end 114.8483 67.01) (width 0.2) (layer "F.Cu") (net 1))
 (segment (start 147.5 80) (end 143.5 84) (width 0.2) (layer "F.Cu") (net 1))
 (segment (start 154.539 71.301) (end 154 71.301) (width 0.2) (layer "F.Cu") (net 1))
 (segment (start 129.7768 68.165) (end 118.0078 68.165) (width 0.2) (layer "F.Cu") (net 1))
 (segment (start 147.5 58) (end 147.5 61.199) (width 0.2) (layer "F.Cu") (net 1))
 (segment (start 155.301 69.4611) (end 155.301 70.5389) (width 0.2) (layer "F.Cu") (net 1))
 (segment (start 114.8483 67.01) (end 113.6184 65.7801) (width 0.2) (layer "F.Cu") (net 1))
 (segment (start 116.5759 67.01) (end 116 67.01) (width 0.2) (layer "F.Cu") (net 1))
 (segment (start 118.0078 68.165) (end 117.1517 67.3089) (width 0.2) (layer "F.Cu") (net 1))
 (segment (start 155.301 70.5389) (end 154.539 71.301) (width 0.2) (layer "F.Cu") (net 1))
 (segment (start 143.5 84) (end 137.5 84) (width 0.2) (layer "F.Cu") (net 1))
 (segment (start 154 71.301) (end 154 73) (width 0.2) (layer "F.Cu") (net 1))
 (segment (start 147.5 61.199) (end 148.039 61.199) (width 0.2) (layer "F.Cu") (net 1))
 (segment (start 147.5 73) (end 154 73) (width 0.2) (layer "F.Cu") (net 1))
 (segment (start 148.1505 64.8495) (end 133.0923 64.8495) (width 0.2) (layer "F.Cu") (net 1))
 (segment (start 148.1505 64.8495) (end 147.5 65.5) (width 0.2) (layer "F.Cu") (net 1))
 (segment (start 117.1517 67.3089) (end 117.1517 67.01) (width 0.2) (layer "F.Cu") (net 1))
 (segment (start 148.801 61.9611) (end 148.801 64.199) (width 0.2) (layer "F.Cu") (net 1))
 (segment (start 154 80) (end 147.5 80) (width 0.2) (layer "F.Cu") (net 1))
 (segment (start 154.539 68.699) (end 155.301 69.4611) (width 0.2) (layer "F.Cu") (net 1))
 (segment (start 116.5759 67.01) (end 117.1517 67.01) (width 0.2) (layer "F.Cu") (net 1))
 (segment (start 148.801 64.199) (end 148.1505 64.8495) (width 0.2) (layer "F.Cu") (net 1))
 (segment (start 154 73) (end 155.3769 74.3769) (width 0.2) (layer "B.Cu") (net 1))
 (segment (start 155.3769 74.3769) (end 155.3769 78.6231) (width 0.2) (layer "B.Cu") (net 1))
 (segment (start 155.3769 78.6231) (end 154 80) (width 0.2) (layer "B.Cu") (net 1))
 (segment (start 133.0983 84.675) (end 133.0983 84) (width 0.2) (layer "B.Cu") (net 3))
 (segment (start 131 87.5) (end 131 86.7733) (width 0.2) (layer "B.Cu") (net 3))
 (segment (start 134.5 84) (end 133.0983 84) (width 0.2) (layer "B.Cu") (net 3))
 (segment (start 131 86.7733) (end 133.0983 84.675) (width 0.2) (layer "B.Cu") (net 3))
 (segment (start 126.5 84) (end 127.9017 84) (width 0.2) (layer "B.Cu") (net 4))
 (segment (start 130 87.5) (end 130 86.7733) (width 0.2) (layer "B.Cu") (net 4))
 (segment (start 130 86.7733) (end 127.9017 84.675) (width 0.2) (layer "B.Cu") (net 4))
 (segment (start 127.9017 84.675) (end 127.9017 84) (width 0.2) (layer "B.Cu") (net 4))
 (segment (start 140.7733 76.585) (end 138.989 78.3693) (width 0.2) (layer "F.Cu") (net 14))
 (segment (start 141.925 76.585) (end 140.7733 76.585) (width 0.2) (layer "F.Cu") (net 14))
 (segment (start 114.8483 77.6946) (end 114.0322 78.5107) (width 0.2) (layer "F.Cu") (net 14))
 (segment (start 114.8483 77.6946) (end 114.8483 77.17) (width 0.2) (layer "F.Cu") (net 14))
 (segment (start 138.989 78.3693) (end 115.523 78.3693) (width 0.2) (layer "F.Cu") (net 14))
 (segment (start 90.691 78.5107) (end 90.0767 79.125) (width 0.2) (layer "F.Cu") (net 14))
 (segment (start 116 77.17) (end 114.8483 77.17) (width 0.2) (layer "F.Cu") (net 14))
 (segment (start 114.0322 78.5107) (end 90.691 78.5107) (width 0.2) (layer "F.Cu") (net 14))
 (segment (start 115.523 78.3693) (end 114.8483 77.6946) (width 0.2) (layer "F.Cu") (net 14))
 (segment (start 88.925 79.125) (end 90.0767 79.125) (width 0.2) (layer "F.Cu") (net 14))
 (segment (start 118.54 77.17) (end 117.3883 77.17) (width 0.2) (layer "F.Cu") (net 13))
 (segment (start 136.26 77.17) (end 118.54 77.17) (width 0.2) (layer "F.Cu") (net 13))
 (segment (start 116.4805 75.9743) (end 90.6874 75.9743) (width 0.2) (layer "F.Cu") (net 13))
 (segment (start 117.3883 77.17) (end 117.3883 76.8821) (width 0.2) (layer "F.Cu") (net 13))
 (segment (start 88.925 76.585) (end 90.0767 76.585) (width 0.2) (layer "F.Cu") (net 13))
 (segment (start 117.3883 76.8821) (end 116.4805 75.9743) (width 0.2) (layer "F.Cu") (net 13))
 (segment (start 90.6874 75.9743) (end 90.0767 76.585) (width 0.2) (layer "F.Cu") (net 13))
 (via (at 136.26 77.17) (size 0.6) (drill 0.3) (layers "F.Cu" "B.Cu") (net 13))
 (segment (start 140.7733 72.6567) (end 136.26 77.17) (width 0.2) (layer "B.Cu") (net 13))
 (segment (start 140.7733 71.505) (end 140.7733 72.6567) (width 0.2) (layer "B.Cu") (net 13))
 (segment (start 141.925 71.505) (end 140.7733 71.505) (width 0.2) (layer "B.Cu") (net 13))
 (segment (start 100.3723 74.63) (end 116 74.63) (width 0.2) (layer "F.Cu") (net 10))
 (via (at 100.3723 74.63) (size 0.6) (drill 0.3) (layers "F.Cu" "B.Cu") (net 10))
 (segment (start 99.0086 73.2663) (end 100.3723 74.63) (width 0.2) (layer "B.Cu") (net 10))
 (segment (start 88.925 68.965) (end 90.0767 68.965) (width 0.2) (layer "B.Cu") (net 10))
 (segment (start 94.378 73.2663) (end 99.0086 73.2663) (width 0.2) (layer "B.Cu") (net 10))
 (segment (start 90.0767 68.965) (end 94.378 73.2663) (width 0.2) (layer "B.Cu") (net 10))
 (segment (start 139.9739 73.2456) (end 101.3512 73.2456) (width 0.2) (layer "F.Cu") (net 17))
 (segment (start 140.7733 74.045) (end 139.9739 73.2456) (width 0.2) (layer "F.Cu") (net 17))
 (segment (start 141.925 74.045) (end 140.7733 74.045) (width 0.2) (layer "F.Cu") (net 17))
 (via (at 101.3512 73.2456) (size 0.6) (drill 0.3) (layers "F.Cu" "B.Cu") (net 17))
 (segment (start 98.22 68.1617) (end 98.5079 68.1617) (width 0.2) (layer "B.Cu") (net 17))
 (segment (start 98.22 67.01) (end 98.22 68.1617) (width 0.2) (layer "B.Cu") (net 17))
 (segment (start 98.5079 68.1617) (end 101.3512 71.005) (width 0.2) (layer "B.Cu") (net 17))
 (segment (start 101.3512 71.005) (end 101.3512 73.2456) (width 0.2) (layer "B.Cu") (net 17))
 (segment (start 141.925 68.965) (end 140.7733 68.965) (width 0.2) (layer "F.Cu") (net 16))
 (segment (start 101.9117 69.55) (end 103.074 70.7123) (width 0.2) (layer "F.Cu") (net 16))
 (segment (start 103.074 70.7123) (end 139.026 70.7123) (width 0.2) (layer "F.Cu") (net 16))
 (segment (start 98.22 69.55) (end 101.9117 69.55) (width 0.2) (layer "F.Cu") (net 16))
 (segment (start 139.026 70.7123) (end 140.7733 68.965) (width 0.2) (layer "F.Cu") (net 16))
 (segment (start 100.3477 72.09) (end 116 72.09) (width 0.2) (layer "F.Cu") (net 11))
 (segment (start 99.1508 70.8931) (end 100.3477 72.09) (width 0.2) (layer "F.Cu") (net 11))
 (segment (start 90.6886 70.8931) (end 99.1508 70.8931) (width 0.2) (layer "F.Cu") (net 11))
 (segment (start 88.925 71.505) (end 90.0767 71.505) (width 0.2) (layer "F.Cu") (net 11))
 (segment (start 90.0767 71.505) (end 90.6886 70.8931) (width 0.2) (layer "F.Cu") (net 11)))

